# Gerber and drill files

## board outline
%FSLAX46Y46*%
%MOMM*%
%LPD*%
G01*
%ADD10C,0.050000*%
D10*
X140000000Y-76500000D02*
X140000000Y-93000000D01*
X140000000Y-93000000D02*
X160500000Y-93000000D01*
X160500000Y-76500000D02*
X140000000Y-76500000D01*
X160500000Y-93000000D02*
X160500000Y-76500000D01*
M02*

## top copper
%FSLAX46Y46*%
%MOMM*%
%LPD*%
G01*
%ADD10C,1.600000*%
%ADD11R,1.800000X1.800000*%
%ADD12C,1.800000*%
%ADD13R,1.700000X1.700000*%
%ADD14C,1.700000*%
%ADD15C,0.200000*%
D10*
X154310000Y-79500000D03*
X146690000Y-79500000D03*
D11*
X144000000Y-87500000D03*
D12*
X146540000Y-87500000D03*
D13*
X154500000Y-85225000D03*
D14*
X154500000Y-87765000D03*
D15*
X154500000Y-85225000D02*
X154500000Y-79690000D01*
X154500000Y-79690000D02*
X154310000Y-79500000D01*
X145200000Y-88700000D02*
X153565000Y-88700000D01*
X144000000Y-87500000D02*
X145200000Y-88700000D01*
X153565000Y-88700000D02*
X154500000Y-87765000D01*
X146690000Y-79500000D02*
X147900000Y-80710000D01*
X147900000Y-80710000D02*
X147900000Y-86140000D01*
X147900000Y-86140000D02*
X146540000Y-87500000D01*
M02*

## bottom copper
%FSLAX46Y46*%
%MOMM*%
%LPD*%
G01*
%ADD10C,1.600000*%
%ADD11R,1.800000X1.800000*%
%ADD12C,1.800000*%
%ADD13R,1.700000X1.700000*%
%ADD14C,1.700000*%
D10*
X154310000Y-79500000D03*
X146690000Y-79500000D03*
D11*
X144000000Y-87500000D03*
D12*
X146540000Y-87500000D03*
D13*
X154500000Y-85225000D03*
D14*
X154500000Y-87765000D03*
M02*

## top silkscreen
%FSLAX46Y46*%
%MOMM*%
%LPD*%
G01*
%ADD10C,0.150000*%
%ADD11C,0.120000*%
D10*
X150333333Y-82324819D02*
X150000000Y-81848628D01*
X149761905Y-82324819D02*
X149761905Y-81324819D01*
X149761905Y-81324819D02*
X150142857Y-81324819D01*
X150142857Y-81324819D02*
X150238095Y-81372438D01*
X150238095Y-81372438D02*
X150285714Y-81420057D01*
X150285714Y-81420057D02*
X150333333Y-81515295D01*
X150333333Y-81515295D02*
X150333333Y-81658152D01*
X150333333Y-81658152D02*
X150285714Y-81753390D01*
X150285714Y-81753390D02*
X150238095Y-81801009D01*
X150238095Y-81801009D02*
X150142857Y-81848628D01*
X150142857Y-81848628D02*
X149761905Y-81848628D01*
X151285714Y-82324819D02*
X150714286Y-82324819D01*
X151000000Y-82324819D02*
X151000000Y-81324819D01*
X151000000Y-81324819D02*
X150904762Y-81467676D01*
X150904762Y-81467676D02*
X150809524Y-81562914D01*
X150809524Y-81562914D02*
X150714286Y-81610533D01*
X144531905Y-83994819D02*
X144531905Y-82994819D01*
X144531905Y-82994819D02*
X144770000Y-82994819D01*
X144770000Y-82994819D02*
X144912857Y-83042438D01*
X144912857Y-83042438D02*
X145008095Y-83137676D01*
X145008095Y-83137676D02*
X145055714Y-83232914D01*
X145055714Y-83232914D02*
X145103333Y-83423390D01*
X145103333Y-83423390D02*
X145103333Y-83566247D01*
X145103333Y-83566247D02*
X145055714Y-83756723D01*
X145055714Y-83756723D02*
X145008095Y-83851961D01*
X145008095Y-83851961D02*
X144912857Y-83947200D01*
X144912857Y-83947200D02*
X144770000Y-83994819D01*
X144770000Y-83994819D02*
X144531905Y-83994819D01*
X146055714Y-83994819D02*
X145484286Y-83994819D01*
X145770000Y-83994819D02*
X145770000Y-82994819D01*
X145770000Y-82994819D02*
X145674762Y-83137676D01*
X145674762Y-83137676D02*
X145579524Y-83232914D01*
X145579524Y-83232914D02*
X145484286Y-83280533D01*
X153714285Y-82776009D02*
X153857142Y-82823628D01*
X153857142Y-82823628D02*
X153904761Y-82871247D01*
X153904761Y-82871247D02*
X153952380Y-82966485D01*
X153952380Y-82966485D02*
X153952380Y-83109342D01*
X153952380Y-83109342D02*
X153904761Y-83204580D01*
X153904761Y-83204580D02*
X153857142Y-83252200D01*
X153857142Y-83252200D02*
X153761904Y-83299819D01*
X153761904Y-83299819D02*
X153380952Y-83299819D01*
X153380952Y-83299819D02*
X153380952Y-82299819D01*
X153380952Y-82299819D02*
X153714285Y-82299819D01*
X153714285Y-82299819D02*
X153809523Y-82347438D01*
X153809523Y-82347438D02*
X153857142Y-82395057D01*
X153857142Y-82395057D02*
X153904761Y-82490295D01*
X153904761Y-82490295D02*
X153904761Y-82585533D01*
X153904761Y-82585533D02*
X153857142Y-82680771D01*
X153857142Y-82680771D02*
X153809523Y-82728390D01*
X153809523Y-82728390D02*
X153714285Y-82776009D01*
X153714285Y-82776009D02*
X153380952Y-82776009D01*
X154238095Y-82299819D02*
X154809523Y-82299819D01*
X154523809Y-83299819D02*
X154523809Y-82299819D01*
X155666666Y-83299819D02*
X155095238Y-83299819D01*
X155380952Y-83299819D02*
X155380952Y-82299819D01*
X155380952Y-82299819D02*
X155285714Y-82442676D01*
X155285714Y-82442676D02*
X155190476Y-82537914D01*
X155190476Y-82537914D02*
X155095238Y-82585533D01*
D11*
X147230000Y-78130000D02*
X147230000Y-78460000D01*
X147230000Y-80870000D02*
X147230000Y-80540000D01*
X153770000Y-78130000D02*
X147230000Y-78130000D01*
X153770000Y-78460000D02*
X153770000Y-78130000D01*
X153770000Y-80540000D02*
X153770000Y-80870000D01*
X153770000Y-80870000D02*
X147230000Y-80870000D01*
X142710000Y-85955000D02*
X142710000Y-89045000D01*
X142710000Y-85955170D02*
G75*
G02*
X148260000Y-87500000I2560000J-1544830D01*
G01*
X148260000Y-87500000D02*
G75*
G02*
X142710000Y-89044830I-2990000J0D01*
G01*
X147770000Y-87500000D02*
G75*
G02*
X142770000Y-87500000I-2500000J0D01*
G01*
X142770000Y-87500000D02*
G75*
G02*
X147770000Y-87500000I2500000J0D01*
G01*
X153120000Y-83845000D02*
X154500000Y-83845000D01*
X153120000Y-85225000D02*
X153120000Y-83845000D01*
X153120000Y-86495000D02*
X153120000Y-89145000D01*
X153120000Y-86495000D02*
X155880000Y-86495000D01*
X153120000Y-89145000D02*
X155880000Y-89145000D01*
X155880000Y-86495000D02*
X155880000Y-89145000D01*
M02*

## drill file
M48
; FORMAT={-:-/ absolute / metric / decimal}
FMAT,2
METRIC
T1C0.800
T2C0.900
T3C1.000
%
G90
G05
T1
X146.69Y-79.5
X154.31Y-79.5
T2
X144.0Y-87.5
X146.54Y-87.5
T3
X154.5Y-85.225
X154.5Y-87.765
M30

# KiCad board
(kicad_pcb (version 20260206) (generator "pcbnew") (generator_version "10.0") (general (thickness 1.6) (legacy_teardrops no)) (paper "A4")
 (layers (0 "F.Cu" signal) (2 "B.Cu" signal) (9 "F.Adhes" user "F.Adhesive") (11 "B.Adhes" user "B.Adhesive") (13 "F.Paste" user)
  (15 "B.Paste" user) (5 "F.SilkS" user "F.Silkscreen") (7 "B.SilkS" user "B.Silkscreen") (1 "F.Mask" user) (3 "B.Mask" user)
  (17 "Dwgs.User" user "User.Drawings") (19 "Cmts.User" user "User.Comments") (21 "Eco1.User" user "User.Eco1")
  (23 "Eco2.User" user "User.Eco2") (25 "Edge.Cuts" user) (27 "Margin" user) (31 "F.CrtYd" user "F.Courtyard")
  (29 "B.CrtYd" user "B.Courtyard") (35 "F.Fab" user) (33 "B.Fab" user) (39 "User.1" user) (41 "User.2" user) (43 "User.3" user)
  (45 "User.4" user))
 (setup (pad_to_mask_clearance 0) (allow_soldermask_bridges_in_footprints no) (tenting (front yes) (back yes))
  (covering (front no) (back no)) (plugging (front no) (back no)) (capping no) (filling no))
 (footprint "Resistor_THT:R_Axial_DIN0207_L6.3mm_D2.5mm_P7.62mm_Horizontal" (layer "F.Cu") (at 154.31 79.5 180)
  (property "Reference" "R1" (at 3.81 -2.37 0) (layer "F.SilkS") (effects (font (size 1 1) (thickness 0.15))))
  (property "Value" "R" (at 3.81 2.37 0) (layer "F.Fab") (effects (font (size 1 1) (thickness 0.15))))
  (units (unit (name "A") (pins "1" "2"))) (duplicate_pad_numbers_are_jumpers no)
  (fp_line (start 7.08 1.37) (end 7.08 1.04) (stroke (width 0.12) (type solid)) (layer "F.SilkS"))
  (fp_line (start 7.08 -1.37) (end 7.08 -1.04) (stroke (width 0.12) (type solid)) (layer "F.SilkS"))
  (fp_line (start 0.54 1.37) (end 7.08 1.37) (stroke (width 0.12) (type solid)) (layer "F.SilkS"))
  (fp_line (start 0.54 1.04) (end 0.54 1.37) (stroke (width 0.12) (type solid)) (layer "F.SilkS"))
  (fp_line (start 0.54 -1.04) (end 0.54 -1.37) (stroke (width 0.12) (type solid)) (layer "F.SilkS"))
  (fp_line (start 0.54 -1.37) (end 7.08 -1.37) (stroke (width 0.12) (type solid)) (layer "F.SilkS"))
  (pad "1" thru_hole circle (at 0 0 180) (size 1.6 1.6) (drill 0.8) (layers "*.Cu" "*.Mask") (remove_unused_layers no) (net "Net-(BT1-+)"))
  (pad "2" thru_hole circle (at 7.62 0 180) (size 1.6 1.6) (drill 0.8) (layers "*.Cu" "*.Mask") (remove_unused_layers no) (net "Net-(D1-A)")))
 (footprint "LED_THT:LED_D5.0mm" (layer "F.Cu") (at 144 87.5)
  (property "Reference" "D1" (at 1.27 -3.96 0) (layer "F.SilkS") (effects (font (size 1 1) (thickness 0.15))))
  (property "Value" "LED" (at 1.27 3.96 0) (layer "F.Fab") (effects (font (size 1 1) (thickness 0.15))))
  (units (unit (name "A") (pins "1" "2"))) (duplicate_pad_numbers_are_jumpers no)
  (fp_line (start -1.29 -1.545) (end -1.29 1.545) (stroke (width 0.12) (type solid)) (layer "F.SilkS"))
  (fp_arc (start -1.29 -1.54483) (mid 2.071779 -2.880495) (end 4.26 0) (stroke (width 0.12) (type solid)) (layer "F.SilkS"))
  (fp_arc (start 4.26 0) (mid 2.071779 2.880495) (end -1.29 1.54483) (stroke (width 0.12) (type solid)) (layer "F.SilkS"))
  (fp_circle (center 1.27 0) (end 3.77 0) (stroke (width 0.12) (type solid)) (fill no) (layer "F.SilkS"))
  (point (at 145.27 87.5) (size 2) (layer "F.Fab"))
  (pad "1" thru_hole rect (at 0 0) (size 1.8 1.8) (drill 0.9) (layers "*.Cu" "*.Mask") (remove_unused_layers no) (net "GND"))
  (pad "2" thru_hole circle (at 2.54 0) (size 1.8 1.8) (drill 0.9) (layers "*.Cu" "*.Mask") (remove_unused_layers no) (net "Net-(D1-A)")))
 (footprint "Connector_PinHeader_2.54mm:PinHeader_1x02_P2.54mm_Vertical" (layer "F.Cu") (at 154.5 85.225)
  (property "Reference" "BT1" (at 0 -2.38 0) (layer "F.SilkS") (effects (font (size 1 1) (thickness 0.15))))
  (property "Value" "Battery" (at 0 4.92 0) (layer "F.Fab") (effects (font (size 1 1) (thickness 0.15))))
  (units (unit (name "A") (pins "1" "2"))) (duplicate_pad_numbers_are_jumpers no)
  (fp_line (start -1.38 -1.38) (end 0 -1.38) (stroke (width 0.12) (type solid)) (layer "F.SilkS"))
  (fp_line (start -1.38 0) (end -1.38 -1.38) (stroke (width 0.12) (type solid)) (layer "F.SilkS"))
  (fp_line (start -1.38 1.27) (end -1.38 3.92) (stroke (width 0.12) (type solid)) (layer "F.SilkS"))
  (fp_line (start -1.38 1.27) (end 1.38 1.27) (stroke (width 0.12) (type solid)) (layer "F.SilkS"))
  (fp_line (start -1.38 3.92) (end 1.38 3.92) (stroke (width 0.12) (type solid)) (layer "F.SilkS"))
  (fp_line (start 1.38 1.27) (end 1.38 3.92) (stroke (width 0.12) (type solid)) (layer "F.SilkS"))
  (pad "1" thru_hole rect (at 0 0) (size 1.7 1.7) (drill 1) (layers "*.Cu" "*.Mask") (remove_unused_layers no) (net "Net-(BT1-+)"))
  (pad "2" thru_hole circle (at 0 2.54) (size 1.7 1.7) (drill 1) (layers "*.Cu" "*.Mask") (remove_unused_layers no) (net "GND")))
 (gr_line (start 140 76.5) (end 140 93) (stroke (width 0.05) (type default)) (layer "Edge.Cuts"))
 (gr_line (start 140 93) (end 160.5 93) (stroke (width 0.05) (type default)) (layer "Edge.Cuts"))
 (gr_line (start 160.5 76.5) (end 140 76.5) (stroke (width 0.05) (type default)) (layer "Edge.Cuts"))
 (gr_line (start 160.5 93) (end 160.5 76.5) (stroke (width 0.05) (type default)) (layer "Edge.Cuts"))
 (segment (start 154.5 85.225) (end 154.5 79.69) (width 0.2) (layer "F.Cu") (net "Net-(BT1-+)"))
 (segment (start 154.5 79.69) (end 154.31 79.5) (width 0.2) (layer "F.Cu") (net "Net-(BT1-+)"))
 (segment (start 145.2 88.7) (end 153.565 88.7) (width 0.2) (layer "F.Cu") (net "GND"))
 (segment (start 144 87.5) (end 145.2 88.7) (width 0.2) (layer "F.Cu") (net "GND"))
 (segment (start 153.565 88.7) (end 154.5 87.765) (width 0.2) (layer "F.Cu") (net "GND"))
 (segment (start 146.69 79.5) (end 147.9 80.71) (width 0.2) (layer "F.Cu") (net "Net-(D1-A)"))
 (segment (start 147.9 80.71) (end 147.9 86.14) (width 0.2) (layer "F.Cu") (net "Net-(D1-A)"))
 (segment (start 147.9 86.14) (end 146.54 87.5) (width 0.2) (layer "F.Cu") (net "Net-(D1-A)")))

